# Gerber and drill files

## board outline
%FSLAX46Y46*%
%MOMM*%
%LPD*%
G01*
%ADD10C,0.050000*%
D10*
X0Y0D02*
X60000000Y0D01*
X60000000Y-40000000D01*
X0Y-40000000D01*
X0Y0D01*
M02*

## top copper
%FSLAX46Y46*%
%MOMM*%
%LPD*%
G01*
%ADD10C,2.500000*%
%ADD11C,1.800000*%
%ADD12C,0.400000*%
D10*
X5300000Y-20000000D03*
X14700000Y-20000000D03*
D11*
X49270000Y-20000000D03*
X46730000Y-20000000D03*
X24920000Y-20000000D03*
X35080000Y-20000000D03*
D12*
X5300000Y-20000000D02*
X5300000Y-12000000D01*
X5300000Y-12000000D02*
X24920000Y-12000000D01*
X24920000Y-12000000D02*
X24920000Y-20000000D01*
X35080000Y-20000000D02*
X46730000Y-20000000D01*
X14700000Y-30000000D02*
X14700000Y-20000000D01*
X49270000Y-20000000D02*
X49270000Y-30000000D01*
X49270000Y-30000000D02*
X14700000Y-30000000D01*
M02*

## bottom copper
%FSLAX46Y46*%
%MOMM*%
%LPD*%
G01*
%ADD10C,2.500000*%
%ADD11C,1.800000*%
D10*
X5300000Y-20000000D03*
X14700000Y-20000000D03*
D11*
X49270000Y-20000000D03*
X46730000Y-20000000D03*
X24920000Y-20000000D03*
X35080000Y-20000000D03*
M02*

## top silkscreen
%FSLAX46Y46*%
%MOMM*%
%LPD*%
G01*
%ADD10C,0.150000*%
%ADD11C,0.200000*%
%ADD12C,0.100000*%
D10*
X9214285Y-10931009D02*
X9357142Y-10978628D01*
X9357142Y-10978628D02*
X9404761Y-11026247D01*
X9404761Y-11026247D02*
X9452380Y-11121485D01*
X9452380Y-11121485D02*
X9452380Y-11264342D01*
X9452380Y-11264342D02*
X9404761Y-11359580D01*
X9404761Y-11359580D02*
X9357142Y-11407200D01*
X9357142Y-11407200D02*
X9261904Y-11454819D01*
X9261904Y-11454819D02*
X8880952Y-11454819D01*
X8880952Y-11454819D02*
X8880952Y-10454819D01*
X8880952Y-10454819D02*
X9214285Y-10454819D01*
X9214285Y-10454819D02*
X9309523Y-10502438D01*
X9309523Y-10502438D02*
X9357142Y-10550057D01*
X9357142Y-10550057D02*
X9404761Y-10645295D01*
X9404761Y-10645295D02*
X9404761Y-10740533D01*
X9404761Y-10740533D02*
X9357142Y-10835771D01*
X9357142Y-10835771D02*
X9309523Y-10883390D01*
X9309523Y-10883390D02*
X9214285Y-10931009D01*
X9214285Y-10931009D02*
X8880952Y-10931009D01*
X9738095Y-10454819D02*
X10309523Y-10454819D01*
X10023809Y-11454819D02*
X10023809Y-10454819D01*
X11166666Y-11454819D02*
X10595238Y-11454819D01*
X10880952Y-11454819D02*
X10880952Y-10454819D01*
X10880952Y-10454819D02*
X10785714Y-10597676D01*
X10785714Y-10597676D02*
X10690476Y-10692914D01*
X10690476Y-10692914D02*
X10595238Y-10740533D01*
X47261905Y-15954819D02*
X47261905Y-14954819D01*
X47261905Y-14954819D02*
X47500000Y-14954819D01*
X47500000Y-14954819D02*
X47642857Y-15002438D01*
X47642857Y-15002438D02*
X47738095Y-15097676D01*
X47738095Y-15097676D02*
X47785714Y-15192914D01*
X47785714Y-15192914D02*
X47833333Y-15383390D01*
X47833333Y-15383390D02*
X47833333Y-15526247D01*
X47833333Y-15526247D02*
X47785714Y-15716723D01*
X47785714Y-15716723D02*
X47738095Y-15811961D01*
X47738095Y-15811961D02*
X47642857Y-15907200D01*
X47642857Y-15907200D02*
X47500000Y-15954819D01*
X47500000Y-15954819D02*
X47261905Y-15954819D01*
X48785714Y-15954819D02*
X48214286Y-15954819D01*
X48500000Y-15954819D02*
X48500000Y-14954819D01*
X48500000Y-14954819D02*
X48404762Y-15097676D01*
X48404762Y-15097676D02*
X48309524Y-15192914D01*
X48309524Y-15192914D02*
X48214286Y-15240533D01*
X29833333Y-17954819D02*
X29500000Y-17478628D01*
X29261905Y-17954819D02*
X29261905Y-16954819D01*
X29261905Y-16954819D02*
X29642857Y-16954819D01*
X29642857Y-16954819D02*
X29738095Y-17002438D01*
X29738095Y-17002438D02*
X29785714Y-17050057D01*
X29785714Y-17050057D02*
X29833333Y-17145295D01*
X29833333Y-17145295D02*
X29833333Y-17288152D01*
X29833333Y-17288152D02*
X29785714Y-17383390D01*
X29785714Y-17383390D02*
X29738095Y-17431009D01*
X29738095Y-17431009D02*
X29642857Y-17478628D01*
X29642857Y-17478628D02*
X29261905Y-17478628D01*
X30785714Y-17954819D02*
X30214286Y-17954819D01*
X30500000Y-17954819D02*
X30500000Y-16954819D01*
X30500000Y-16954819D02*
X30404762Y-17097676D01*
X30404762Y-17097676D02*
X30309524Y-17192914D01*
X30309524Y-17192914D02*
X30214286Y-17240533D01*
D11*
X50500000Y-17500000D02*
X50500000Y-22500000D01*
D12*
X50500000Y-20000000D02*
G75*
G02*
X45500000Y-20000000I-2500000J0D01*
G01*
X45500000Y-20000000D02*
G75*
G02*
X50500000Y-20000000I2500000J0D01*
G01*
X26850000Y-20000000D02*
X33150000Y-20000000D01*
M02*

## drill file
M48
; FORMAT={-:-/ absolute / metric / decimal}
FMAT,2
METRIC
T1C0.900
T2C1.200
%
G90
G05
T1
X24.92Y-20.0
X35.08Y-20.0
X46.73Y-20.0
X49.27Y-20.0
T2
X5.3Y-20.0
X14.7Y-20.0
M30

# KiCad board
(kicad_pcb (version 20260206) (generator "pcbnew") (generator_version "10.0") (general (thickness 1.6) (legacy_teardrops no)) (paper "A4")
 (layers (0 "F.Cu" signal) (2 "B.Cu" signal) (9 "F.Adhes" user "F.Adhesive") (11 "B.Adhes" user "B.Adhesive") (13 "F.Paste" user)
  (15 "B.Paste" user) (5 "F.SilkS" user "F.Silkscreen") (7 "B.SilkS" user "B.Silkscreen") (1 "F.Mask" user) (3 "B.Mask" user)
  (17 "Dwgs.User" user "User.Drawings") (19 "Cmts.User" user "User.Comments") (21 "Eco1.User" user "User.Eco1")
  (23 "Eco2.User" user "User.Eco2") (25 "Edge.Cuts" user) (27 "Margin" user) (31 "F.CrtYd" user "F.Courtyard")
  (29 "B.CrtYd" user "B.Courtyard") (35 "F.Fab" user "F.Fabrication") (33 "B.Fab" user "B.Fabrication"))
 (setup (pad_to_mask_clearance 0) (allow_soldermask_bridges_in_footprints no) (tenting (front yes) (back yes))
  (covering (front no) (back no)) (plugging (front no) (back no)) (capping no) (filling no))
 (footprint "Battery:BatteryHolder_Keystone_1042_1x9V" (layer "F.Cu") (at 10 20)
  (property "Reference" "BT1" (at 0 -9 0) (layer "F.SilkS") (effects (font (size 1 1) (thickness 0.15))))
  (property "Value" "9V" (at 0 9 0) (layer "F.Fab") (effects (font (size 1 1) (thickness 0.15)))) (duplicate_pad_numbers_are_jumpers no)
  (pad "+" thru_hole circle (at -4.7 0) (size 2.5 2.5) (drill 1.2) (layers "*.Cu" "*.Mask") (remove_unused_layers no) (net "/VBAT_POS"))
  (pad "-" thru_hole circle (at 4.7 0) (size 2.5 2.5) (drill 1.2) (layers "*.Cu" "*.Mask") (remove_unused_layers no) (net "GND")))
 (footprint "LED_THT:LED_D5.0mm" (layer "F.Cu") (at 48 20)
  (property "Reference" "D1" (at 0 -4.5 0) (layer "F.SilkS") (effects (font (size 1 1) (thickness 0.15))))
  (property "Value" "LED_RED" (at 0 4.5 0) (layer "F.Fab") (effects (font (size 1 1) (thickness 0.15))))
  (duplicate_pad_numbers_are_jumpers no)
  (fp_line (start 2.5 -2.5) (end 2.5 2.5) (stroke (width 0.2) (type default)) (layer "F.SilkS"))
  (fp_circle (center 0 0) (end 2.5 0) (stroke (width 0.1) (type default)) (fill no) (layer "F.SilkS"))
  (pad "1" thru_hole circle (at 1.27 0) (size 1.8 1.8) (drill 0.9) (layers "*.Cu" "*.Mask") (remove_unused_layers no) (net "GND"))
  (pad "2" thru_hole circle (at -1.27 0) (size 1.8 1.8) (drill 0.9) (layers "*.Cu" "*.Mask") (remove_unused_layers no) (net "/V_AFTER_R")))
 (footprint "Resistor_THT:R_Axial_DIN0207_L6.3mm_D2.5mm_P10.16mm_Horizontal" (layer "F.Cu") (at 30 20)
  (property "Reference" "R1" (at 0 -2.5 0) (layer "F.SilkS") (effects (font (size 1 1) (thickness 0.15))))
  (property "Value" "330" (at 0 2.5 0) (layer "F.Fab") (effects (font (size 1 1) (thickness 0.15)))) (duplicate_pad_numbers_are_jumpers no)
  (fp_line (start -3.15 0) (end 3.15 0) (stroke (width 0.1) (type default)) (layer "F.SilkS"))
  (pad "1" thru_hole circle (at -5.08 0) (size 1.8 1.8) (drill 0.9) (layers "*.Cu" "*.Mask") (remove_unused_layers no) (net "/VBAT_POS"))
  (pad "2" thru_hole circle (at 5.08 0) (size 1.8 1.8) (drill 0.9) (layers "*.Cu" "*.Mask") (remove_unused_layers no) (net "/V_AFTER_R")))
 (gr_rect (start 0 0) (end 60 40) (stroke (width 0.05) (type default)) (fill no) (layer "Edge.Cuts"))
 (segment (start 5.3 20) (end 5.3 12) (width 0.4) (layer "F.Cu") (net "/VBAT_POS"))
 (segment (start 5.3 12) (end 24.92 12) (width 0.4) (layer "F.Cu") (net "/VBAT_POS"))
 (segment (start 24.92 12) (end 24.92 20) (width 0.4) (layer "F.Cu") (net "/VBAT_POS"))
 (segment (start 35.08 20) (end 46.73 20) (width 0.4) (layer "F.Cu") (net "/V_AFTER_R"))
 (segment (start 14.7 30) (end 14.7 20) (width 0.4) (layer "F.Cu") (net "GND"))
 (segment (start 49.27 20) (end 49.27 30) (width 0.4) (layer "F.Cu") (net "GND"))
 (segment (start 49.27 30) (end 14.7 30) (width 0.4) (layer "F.Cu") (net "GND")))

